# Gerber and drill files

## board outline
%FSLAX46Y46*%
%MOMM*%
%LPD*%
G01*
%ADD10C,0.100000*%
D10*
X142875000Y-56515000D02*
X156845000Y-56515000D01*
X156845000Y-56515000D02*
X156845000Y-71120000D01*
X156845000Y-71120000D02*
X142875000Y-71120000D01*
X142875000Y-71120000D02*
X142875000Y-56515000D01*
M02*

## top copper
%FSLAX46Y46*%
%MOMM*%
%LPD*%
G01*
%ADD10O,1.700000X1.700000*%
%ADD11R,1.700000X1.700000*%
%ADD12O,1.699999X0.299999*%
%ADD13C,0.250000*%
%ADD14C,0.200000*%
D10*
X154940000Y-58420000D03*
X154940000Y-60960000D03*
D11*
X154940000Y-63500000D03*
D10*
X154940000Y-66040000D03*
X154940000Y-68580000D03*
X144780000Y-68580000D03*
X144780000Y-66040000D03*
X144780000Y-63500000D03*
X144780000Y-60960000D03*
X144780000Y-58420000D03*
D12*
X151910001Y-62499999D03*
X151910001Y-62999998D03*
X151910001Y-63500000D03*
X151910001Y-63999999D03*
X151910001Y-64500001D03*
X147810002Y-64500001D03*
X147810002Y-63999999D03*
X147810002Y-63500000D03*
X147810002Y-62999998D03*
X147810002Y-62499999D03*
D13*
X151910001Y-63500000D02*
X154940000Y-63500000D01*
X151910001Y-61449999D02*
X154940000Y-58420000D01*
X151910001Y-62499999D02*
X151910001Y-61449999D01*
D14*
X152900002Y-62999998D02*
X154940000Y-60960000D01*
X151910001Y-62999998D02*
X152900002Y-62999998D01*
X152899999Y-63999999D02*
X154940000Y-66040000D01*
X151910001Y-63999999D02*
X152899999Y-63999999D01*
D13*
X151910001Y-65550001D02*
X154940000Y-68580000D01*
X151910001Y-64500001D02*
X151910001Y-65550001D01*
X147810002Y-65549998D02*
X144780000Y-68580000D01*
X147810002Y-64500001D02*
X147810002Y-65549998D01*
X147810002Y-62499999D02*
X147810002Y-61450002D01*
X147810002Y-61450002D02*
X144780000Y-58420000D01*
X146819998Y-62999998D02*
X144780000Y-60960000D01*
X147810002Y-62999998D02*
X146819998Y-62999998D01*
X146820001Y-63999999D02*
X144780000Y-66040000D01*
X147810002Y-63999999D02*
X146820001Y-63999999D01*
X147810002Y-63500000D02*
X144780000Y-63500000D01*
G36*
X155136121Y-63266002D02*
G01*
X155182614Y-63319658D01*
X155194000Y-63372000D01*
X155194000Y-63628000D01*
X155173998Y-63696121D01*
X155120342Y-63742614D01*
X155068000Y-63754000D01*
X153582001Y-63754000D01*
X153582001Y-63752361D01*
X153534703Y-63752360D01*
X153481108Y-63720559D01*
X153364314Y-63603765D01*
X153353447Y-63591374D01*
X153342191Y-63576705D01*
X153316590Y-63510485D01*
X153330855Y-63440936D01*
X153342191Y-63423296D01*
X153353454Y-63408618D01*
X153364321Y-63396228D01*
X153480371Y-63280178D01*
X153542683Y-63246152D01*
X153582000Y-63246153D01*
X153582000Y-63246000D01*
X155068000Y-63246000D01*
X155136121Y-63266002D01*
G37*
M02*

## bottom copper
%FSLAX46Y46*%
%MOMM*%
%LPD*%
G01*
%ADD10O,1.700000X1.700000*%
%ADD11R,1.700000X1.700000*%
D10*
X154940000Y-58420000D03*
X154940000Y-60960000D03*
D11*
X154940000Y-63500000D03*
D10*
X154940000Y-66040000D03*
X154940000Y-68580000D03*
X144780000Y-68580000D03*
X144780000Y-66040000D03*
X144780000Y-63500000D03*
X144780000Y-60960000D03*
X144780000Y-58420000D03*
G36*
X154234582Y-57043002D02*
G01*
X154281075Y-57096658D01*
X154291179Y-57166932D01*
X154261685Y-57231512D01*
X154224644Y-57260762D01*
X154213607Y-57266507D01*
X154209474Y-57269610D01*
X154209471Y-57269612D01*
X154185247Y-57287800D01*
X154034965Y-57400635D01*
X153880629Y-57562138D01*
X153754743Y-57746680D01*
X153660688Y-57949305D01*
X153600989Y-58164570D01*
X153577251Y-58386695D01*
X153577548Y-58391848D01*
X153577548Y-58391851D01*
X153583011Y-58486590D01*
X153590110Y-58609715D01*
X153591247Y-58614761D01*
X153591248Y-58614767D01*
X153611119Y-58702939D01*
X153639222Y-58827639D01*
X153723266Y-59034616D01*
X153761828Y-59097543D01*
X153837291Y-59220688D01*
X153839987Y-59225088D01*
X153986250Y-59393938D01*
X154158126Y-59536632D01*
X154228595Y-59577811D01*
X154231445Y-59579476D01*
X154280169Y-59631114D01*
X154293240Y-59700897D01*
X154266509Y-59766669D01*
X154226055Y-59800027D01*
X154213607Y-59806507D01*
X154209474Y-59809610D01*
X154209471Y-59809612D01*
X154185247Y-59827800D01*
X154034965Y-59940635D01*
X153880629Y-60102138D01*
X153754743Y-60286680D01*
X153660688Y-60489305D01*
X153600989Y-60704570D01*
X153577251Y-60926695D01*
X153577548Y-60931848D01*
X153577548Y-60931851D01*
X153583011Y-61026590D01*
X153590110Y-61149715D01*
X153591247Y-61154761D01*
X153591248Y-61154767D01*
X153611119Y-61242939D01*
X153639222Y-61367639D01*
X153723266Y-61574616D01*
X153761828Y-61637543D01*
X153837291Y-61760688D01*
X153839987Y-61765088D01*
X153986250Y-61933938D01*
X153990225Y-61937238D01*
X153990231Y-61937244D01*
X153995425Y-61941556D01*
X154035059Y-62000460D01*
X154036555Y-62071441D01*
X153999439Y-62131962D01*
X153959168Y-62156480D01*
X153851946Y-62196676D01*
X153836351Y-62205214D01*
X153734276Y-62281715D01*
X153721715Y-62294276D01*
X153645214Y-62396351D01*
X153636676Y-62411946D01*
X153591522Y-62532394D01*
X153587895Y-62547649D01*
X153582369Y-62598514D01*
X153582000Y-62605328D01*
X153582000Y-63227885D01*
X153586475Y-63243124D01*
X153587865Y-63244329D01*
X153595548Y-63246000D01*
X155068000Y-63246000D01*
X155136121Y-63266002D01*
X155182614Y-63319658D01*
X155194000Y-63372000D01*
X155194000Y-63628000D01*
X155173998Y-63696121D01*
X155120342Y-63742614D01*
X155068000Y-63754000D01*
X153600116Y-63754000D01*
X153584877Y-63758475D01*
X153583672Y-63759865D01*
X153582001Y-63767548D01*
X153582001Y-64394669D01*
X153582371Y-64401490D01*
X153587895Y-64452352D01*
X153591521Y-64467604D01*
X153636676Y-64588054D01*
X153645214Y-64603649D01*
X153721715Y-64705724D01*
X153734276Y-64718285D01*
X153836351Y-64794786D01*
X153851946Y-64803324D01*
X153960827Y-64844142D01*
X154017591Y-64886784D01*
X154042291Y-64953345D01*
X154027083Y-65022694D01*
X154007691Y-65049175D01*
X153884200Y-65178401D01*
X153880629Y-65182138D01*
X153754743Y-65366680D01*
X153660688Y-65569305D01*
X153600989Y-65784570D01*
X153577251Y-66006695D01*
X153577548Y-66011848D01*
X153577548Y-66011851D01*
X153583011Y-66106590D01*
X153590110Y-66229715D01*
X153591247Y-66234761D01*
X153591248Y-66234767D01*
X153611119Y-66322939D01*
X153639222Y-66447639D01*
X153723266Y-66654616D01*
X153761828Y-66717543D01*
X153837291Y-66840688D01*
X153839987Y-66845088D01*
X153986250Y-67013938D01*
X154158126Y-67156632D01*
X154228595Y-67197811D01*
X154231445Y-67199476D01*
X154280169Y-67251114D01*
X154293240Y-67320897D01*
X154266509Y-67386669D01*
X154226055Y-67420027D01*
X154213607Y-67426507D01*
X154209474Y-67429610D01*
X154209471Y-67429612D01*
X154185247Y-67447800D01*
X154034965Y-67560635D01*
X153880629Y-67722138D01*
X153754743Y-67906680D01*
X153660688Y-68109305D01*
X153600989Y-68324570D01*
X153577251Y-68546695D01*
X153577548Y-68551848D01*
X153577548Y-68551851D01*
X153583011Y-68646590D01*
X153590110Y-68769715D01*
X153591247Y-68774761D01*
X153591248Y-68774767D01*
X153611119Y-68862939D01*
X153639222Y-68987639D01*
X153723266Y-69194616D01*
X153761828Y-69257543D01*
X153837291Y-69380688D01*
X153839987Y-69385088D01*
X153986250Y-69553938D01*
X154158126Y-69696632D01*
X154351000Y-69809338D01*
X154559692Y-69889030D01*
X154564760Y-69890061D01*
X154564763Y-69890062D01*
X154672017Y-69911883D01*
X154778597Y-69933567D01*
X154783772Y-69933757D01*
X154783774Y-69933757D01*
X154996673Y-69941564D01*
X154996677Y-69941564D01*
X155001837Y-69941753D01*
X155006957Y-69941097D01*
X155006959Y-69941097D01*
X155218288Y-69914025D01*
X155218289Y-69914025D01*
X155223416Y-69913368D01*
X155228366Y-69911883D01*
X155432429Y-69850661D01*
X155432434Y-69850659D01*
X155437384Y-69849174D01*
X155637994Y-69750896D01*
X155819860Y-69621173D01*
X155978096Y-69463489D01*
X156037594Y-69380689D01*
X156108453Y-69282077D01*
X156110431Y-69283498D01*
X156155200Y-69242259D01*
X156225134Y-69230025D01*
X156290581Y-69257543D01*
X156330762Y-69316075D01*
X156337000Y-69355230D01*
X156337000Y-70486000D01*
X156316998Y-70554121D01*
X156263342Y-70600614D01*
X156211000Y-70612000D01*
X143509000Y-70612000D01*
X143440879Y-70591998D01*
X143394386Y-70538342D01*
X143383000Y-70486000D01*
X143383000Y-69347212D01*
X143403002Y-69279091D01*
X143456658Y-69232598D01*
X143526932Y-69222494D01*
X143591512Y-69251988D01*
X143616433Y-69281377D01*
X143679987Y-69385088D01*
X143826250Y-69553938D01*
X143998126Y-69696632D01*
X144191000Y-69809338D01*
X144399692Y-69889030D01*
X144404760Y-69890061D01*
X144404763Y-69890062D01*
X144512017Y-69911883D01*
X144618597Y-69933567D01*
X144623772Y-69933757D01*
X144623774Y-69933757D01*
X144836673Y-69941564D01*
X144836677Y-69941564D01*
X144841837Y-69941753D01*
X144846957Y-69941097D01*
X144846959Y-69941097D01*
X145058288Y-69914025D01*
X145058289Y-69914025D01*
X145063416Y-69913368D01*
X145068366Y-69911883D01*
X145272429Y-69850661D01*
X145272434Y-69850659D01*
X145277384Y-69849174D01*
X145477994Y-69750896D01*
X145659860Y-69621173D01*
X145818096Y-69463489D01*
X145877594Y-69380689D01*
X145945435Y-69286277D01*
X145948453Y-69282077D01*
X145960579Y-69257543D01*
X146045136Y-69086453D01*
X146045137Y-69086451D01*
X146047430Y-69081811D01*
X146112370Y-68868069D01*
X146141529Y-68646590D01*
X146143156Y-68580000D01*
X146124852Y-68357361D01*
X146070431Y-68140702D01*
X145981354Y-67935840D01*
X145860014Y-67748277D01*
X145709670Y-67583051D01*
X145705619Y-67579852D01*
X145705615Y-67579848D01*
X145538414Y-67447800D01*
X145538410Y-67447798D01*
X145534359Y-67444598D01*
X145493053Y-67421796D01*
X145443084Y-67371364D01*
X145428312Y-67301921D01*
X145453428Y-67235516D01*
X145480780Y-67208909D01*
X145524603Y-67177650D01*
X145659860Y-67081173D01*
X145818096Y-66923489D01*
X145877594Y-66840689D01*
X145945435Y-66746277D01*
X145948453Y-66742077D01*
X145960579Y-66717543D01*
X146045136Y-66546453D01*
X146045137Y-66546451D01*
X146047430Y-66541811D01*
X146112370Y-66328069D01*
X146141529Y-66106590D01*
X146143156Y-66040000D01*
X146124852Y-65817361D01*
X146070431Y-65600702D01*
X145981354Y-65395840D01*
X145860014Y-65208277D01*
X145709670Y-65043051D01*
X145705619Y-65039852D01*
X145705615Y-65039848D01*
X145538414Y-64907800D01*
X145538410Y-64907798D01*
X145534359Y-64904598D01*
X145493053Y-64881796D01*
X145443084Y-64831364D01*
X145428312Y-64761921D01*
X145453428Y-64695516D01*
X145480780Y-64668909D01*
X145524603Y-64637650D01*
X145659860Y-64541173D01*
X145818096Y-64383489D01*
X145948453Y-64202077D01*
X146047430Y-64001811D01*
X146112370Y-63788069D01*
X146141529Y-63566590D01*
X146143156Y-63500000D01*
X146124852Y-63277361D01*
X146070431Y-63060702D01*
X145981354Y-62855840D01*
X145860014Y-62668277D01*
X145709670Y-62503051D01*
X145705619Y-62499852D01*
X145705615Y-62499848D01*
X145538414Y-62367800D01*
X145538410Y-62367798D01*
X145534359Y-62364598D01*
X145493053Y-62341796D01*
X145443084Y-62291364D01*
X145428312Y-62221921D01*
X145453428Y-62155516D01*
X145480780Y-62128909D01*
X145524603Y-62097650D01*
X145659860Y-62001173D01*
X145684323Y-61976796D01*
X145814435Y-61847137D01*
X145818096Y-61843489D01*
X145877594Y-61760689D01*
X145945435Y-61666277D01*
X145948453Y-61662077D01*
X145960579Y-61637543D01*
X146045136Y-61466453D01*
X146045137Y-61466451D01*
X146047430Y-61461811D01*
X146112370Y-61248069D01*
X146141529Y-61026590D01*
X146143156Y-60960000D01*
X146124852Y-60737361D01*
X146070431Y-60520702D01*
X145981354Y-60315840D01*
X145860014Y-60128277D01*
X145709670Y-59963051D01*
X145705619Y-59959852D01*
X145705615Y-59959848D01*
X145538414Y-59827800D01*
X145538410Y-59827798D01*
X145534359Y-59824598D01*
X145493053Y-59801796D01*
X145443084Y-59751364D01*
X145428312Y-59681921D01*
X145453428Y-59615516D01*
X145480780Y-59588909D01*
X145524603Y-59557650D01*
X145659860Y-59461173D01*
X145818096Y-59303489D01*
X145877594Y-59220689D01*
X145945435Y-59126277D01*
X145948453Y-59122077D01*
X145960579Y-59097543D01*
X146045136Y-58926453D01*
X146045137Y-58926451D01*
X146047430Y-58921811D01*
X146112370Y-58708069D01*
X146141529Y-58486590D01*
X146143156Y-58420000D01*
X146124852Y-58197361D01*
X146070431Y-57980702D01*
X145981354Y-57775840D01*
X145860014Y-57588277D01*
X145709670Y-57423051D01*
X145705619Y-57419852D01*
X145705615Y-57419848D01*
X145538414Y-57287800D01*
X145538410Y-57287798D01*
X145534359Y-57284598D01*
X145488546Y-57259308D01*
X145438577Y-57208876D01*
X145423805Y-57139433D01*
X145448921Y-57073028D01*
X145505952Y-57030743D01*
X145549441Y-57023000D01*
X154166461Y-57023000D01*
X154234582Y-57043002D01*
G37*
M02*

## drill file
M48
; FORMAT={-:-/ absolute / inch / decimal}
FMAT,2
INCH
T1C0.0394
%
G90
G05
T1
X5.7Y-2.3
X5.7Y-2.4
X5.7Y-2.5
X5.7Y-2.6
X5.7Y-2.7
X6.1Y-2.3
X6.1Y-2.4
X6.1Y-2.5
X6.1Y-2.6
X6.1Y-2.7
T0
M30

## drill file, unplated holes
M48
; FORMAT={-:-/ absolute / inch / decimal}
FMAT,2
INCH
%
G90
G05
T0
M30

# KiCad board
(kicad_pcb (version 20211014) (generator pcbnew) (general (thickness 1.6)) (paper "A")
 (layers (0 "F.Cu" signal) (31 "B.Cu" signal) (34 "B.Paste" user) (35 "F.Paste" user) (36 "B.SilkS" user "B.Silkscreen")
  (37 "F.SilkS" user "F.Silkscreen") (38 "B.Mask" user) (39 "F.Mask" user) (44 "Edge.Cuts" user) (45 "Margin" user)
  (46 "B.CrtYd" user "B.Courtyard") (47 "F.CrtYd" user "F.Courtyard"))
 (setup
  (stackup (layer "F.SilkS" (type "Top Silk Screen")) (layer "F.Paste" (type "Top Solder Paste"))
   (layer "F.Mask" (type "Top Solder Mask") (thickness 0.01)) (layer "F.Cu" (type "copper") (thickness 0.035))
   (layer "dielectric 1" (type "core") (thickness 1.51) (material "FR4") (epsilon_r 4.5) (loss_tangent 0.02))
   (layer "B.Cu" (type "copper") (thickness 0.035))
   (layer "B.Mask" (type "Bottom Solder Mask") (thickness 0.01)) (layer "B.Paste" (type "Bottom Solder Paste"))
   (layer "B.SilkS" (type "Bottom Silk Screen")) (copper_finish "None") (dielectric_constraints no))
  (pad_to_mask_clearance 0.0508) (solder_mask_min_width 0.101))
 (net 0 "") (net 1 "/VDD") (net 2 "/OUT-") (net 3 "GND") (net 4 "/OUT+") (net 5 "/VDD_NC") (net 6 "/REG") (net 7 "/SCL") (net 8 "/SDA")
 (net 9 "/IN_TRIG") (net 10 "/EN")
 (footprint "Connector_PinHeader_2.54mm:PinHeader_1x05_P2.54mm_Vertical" (layer "F.Cu") (at 154.94 58.42)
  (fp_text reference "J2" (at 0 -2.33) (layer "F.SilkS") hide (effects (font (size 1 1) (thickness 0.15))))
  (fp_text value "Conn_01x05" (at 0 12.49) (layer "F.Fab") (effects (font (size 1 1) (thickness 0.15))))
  (pad "1" thru_hole oval (at 0 0) (size 1.7 1.7) (drill 1) (layers *.Cu *.Mask) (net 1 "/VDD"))
  (pad "2" thru_hole oval (at 0 2.54) (size 1.7 1.7) (drill 1) (layers *.Cu *.Mask) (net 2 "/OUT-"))
  (pad "3" thru_hole rect (at 0 5.08) (size 1.7 1.7) (drill 1) (layers *.Cu *.Mask) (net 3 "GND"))
  (pad "4" thru_hole oval (at 0 7.62) (size 1.7 1.7) (drill 1) (layers *.Cu *.Mask) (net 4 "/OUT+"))
  (pad "5" thru_hole oval (at 0 10.16) (size 1.7 1.7) (drill 1) (layers *.Cu *.Mask) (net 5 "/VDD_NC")))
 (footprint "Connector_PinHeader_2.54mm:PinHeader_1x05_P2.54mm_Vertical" (layer "F.Cu") (at 144.78 58.42)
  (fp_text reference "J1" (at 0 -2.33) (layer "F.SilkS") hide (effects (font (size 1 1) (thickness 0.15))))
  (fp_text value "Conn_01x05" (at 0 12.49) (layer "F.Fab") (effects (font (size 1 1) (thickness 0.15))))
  (pad "1" thru_hole oval (at 0 0) (size 1.7 1.7) (drill 1) (layers *.Cu *.Mask) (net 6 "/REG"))
  (pad "2" thru_hole oval (at 0 2.54) (size 1.7 1.7) (drill 1) (layers *.Cu *.Mask) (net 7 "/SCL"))
  (pad "3" thru_hole oval (at 0 5.08) (size 1.7 1.7) (drill 1) (layers *.Cu *.Mask) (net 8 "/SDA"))
  (pad "4" thru_hole oval (at 0 7.62) (size 1.7 1.7) (drill 1) (layers *.Cu *.Mask) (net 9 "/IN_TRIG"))
  (pad "5" thru_hole oval (at 0 10.16) (size 1.7 1.7) (drill 1) (layers *.Cu *.Mask) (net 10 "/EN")))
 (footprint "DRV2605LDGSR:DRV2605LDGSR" (layer "F.Cu") (at 149.86 63.5)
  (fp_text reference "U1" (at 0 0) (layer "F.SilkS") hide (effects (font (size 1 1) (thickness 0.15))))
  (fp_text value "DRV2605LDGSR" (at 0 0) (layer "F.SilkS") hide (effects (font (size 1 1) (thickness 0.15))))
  (pad "1" smd oval (at -2.049998 -1.000001 90) (size 0.299999 1.699999) (layers "F.Cu" "F.Paste" "F.Mask") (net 6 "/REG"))
  (pad "2" smd oval (at -2.049998 -0.500002 90) (size 0.299999 1.699999) (layers "F.Cu" "F.Paste" "F.Mask") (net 7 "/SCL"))
  (pad "3" smd oval (at -2.049998 0 90) (size 0.299999 1.699999) (layers "F.Cu" "F.Paste" "F.Mask") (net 8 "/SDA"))
  (pad "4" smd oval (at -2.049998 0.499999 90) (size 0.299999 1.699999) (layers "F.Cu" "F.Paste" "F.Mask") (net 9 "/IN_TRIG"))
  (pad "5" smd oval (at -2.049998 1.000001 90) (size 0.299999 1.699999) (layers "F.Cu" "F.Paste" "F.Mask") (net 10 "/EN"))
  (pad "6" smd oval (at 2.050001 1.000001 90) (size 0.299999 1.699999) (layers "F.Cu" "F.Paste" "F.Mask") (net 5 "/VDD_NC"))
  (pad "7" smd oval (at 2.050001 0.499999 90) (size 0.299999 1.699999) (layers "F.Cu" "F.Paste" "F.Mask") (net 4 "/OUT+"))
  (pad "8" smd oval (at 2.050001 0 90) (size 0.299999 1.699999) (layers "F.Cu" "F.Paste" "F.Mask") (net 3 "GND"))
  (pad "9" smd oval (at 2.050001 -0.500002 90) (size 0.299999 1.699999) (layers "F.Cu" "F.Paste" "F.Mask") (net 2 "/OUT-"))
  (pad "10" smd oval (at 2.050001 -1.000001 90) (size 0.299999 1.699999) (layers "F.Cu" "F.Paste" "F.Mask") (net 1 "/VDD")))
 (gr_rect (start 142.875 56.515) (end 156.845 71.12) (layer "Edge.Cuts") (width 0.1) (fill none))
 (segment (start 147.810002 61.450002) (end 144.78 58.42) (width 0.25) (layer "F.Cu") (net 6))
 (segment (start 147.810002 62.499999) (end 147.810002 61.450002) (width 0.25) (layer "F.Cu") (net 6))
 (segment (start 146.819998 62.999998) (end 144.78 60.96) (width 0.25) (layer "F.Cu") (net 7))
 (segment (start 147.810002 62.999998) (end 146.819998 62.999998) (width 0.25) (layer "F.Cu") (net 7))
 (segment (start 147.810002 63.5) (end 144.78 63.5) (width 0.25) (layer "F.Cu") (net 8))
 (segment (start 147.810002 63.999999) (end 146.820001 63.999999) (width 0.25) (layer "F.Cu") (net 9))
 (segment (start 146.820001 63.999999) (end 144.78 66.04) (width 0.25) (layer "F.Cu") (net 9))
 (segment (start 147.810002 64.500001) (end 147.810002 65.549998) (width 0.25) (layer "F.Cu") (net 10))
 (segment (start 147.810002 65.549998) (end 144.78 68.58) (width 0.25) (layer "F.Cu") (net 10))
 (segment (start 151.910001 61.449999) (end 154.94 58.42) (width 0.25) (layer "F.Cu") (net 1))
 (segment (start 151.910001 62.499999) (end 151.910001 61.449999) (width 0.25) (layer "F.Cu") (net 1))
 (segment (start 151.910001 62.999998) (end 152.900002 62.999998) (width 0.2) (layer "F.Cu") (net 2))
 (segment (start 152.900002 62.999998) (end 154.94 60.96) (width 0.2) (layer "F.Cu") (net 2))
 (segment (start 151.910001 63.5) (end 154.94 63.5) (width 0.25) (layer "F.Cu") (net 3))
 (segment (start 152.899999 63.999999) (end 154.94 66.04) (width 0.2) (layer "F.Cu") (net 4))
 (segment (start 151.910001 63.999999) (end 152.899999 63.999999) (width 0.2) (layer "F.Cu") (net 4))
 (segment (start 151.910001 65.550001) (end 154.94 68.58) (width 0.25) (layer "F.Cu") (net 5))
 (segment (start 151.910001 64.500001) (end 151.910001 65.550001) (width 0.25) (layer "F.Cu") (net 5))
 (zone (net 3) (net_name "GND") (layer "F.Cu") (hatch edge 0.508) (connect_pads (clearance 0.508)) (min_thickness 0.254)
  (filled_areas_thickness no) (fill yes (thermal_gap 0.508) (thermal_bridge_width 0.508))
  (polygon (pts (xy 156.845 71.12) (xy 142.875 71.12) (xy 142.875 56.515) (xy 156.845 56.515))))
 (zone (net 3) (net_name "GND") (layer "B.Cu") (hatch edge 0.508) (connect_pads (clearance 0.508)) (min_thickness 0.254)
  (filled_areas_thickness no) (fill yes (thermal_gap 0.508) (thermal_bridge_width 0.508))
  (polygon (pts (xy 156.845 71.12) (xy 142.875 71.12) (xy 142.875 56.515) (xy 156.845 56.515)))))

